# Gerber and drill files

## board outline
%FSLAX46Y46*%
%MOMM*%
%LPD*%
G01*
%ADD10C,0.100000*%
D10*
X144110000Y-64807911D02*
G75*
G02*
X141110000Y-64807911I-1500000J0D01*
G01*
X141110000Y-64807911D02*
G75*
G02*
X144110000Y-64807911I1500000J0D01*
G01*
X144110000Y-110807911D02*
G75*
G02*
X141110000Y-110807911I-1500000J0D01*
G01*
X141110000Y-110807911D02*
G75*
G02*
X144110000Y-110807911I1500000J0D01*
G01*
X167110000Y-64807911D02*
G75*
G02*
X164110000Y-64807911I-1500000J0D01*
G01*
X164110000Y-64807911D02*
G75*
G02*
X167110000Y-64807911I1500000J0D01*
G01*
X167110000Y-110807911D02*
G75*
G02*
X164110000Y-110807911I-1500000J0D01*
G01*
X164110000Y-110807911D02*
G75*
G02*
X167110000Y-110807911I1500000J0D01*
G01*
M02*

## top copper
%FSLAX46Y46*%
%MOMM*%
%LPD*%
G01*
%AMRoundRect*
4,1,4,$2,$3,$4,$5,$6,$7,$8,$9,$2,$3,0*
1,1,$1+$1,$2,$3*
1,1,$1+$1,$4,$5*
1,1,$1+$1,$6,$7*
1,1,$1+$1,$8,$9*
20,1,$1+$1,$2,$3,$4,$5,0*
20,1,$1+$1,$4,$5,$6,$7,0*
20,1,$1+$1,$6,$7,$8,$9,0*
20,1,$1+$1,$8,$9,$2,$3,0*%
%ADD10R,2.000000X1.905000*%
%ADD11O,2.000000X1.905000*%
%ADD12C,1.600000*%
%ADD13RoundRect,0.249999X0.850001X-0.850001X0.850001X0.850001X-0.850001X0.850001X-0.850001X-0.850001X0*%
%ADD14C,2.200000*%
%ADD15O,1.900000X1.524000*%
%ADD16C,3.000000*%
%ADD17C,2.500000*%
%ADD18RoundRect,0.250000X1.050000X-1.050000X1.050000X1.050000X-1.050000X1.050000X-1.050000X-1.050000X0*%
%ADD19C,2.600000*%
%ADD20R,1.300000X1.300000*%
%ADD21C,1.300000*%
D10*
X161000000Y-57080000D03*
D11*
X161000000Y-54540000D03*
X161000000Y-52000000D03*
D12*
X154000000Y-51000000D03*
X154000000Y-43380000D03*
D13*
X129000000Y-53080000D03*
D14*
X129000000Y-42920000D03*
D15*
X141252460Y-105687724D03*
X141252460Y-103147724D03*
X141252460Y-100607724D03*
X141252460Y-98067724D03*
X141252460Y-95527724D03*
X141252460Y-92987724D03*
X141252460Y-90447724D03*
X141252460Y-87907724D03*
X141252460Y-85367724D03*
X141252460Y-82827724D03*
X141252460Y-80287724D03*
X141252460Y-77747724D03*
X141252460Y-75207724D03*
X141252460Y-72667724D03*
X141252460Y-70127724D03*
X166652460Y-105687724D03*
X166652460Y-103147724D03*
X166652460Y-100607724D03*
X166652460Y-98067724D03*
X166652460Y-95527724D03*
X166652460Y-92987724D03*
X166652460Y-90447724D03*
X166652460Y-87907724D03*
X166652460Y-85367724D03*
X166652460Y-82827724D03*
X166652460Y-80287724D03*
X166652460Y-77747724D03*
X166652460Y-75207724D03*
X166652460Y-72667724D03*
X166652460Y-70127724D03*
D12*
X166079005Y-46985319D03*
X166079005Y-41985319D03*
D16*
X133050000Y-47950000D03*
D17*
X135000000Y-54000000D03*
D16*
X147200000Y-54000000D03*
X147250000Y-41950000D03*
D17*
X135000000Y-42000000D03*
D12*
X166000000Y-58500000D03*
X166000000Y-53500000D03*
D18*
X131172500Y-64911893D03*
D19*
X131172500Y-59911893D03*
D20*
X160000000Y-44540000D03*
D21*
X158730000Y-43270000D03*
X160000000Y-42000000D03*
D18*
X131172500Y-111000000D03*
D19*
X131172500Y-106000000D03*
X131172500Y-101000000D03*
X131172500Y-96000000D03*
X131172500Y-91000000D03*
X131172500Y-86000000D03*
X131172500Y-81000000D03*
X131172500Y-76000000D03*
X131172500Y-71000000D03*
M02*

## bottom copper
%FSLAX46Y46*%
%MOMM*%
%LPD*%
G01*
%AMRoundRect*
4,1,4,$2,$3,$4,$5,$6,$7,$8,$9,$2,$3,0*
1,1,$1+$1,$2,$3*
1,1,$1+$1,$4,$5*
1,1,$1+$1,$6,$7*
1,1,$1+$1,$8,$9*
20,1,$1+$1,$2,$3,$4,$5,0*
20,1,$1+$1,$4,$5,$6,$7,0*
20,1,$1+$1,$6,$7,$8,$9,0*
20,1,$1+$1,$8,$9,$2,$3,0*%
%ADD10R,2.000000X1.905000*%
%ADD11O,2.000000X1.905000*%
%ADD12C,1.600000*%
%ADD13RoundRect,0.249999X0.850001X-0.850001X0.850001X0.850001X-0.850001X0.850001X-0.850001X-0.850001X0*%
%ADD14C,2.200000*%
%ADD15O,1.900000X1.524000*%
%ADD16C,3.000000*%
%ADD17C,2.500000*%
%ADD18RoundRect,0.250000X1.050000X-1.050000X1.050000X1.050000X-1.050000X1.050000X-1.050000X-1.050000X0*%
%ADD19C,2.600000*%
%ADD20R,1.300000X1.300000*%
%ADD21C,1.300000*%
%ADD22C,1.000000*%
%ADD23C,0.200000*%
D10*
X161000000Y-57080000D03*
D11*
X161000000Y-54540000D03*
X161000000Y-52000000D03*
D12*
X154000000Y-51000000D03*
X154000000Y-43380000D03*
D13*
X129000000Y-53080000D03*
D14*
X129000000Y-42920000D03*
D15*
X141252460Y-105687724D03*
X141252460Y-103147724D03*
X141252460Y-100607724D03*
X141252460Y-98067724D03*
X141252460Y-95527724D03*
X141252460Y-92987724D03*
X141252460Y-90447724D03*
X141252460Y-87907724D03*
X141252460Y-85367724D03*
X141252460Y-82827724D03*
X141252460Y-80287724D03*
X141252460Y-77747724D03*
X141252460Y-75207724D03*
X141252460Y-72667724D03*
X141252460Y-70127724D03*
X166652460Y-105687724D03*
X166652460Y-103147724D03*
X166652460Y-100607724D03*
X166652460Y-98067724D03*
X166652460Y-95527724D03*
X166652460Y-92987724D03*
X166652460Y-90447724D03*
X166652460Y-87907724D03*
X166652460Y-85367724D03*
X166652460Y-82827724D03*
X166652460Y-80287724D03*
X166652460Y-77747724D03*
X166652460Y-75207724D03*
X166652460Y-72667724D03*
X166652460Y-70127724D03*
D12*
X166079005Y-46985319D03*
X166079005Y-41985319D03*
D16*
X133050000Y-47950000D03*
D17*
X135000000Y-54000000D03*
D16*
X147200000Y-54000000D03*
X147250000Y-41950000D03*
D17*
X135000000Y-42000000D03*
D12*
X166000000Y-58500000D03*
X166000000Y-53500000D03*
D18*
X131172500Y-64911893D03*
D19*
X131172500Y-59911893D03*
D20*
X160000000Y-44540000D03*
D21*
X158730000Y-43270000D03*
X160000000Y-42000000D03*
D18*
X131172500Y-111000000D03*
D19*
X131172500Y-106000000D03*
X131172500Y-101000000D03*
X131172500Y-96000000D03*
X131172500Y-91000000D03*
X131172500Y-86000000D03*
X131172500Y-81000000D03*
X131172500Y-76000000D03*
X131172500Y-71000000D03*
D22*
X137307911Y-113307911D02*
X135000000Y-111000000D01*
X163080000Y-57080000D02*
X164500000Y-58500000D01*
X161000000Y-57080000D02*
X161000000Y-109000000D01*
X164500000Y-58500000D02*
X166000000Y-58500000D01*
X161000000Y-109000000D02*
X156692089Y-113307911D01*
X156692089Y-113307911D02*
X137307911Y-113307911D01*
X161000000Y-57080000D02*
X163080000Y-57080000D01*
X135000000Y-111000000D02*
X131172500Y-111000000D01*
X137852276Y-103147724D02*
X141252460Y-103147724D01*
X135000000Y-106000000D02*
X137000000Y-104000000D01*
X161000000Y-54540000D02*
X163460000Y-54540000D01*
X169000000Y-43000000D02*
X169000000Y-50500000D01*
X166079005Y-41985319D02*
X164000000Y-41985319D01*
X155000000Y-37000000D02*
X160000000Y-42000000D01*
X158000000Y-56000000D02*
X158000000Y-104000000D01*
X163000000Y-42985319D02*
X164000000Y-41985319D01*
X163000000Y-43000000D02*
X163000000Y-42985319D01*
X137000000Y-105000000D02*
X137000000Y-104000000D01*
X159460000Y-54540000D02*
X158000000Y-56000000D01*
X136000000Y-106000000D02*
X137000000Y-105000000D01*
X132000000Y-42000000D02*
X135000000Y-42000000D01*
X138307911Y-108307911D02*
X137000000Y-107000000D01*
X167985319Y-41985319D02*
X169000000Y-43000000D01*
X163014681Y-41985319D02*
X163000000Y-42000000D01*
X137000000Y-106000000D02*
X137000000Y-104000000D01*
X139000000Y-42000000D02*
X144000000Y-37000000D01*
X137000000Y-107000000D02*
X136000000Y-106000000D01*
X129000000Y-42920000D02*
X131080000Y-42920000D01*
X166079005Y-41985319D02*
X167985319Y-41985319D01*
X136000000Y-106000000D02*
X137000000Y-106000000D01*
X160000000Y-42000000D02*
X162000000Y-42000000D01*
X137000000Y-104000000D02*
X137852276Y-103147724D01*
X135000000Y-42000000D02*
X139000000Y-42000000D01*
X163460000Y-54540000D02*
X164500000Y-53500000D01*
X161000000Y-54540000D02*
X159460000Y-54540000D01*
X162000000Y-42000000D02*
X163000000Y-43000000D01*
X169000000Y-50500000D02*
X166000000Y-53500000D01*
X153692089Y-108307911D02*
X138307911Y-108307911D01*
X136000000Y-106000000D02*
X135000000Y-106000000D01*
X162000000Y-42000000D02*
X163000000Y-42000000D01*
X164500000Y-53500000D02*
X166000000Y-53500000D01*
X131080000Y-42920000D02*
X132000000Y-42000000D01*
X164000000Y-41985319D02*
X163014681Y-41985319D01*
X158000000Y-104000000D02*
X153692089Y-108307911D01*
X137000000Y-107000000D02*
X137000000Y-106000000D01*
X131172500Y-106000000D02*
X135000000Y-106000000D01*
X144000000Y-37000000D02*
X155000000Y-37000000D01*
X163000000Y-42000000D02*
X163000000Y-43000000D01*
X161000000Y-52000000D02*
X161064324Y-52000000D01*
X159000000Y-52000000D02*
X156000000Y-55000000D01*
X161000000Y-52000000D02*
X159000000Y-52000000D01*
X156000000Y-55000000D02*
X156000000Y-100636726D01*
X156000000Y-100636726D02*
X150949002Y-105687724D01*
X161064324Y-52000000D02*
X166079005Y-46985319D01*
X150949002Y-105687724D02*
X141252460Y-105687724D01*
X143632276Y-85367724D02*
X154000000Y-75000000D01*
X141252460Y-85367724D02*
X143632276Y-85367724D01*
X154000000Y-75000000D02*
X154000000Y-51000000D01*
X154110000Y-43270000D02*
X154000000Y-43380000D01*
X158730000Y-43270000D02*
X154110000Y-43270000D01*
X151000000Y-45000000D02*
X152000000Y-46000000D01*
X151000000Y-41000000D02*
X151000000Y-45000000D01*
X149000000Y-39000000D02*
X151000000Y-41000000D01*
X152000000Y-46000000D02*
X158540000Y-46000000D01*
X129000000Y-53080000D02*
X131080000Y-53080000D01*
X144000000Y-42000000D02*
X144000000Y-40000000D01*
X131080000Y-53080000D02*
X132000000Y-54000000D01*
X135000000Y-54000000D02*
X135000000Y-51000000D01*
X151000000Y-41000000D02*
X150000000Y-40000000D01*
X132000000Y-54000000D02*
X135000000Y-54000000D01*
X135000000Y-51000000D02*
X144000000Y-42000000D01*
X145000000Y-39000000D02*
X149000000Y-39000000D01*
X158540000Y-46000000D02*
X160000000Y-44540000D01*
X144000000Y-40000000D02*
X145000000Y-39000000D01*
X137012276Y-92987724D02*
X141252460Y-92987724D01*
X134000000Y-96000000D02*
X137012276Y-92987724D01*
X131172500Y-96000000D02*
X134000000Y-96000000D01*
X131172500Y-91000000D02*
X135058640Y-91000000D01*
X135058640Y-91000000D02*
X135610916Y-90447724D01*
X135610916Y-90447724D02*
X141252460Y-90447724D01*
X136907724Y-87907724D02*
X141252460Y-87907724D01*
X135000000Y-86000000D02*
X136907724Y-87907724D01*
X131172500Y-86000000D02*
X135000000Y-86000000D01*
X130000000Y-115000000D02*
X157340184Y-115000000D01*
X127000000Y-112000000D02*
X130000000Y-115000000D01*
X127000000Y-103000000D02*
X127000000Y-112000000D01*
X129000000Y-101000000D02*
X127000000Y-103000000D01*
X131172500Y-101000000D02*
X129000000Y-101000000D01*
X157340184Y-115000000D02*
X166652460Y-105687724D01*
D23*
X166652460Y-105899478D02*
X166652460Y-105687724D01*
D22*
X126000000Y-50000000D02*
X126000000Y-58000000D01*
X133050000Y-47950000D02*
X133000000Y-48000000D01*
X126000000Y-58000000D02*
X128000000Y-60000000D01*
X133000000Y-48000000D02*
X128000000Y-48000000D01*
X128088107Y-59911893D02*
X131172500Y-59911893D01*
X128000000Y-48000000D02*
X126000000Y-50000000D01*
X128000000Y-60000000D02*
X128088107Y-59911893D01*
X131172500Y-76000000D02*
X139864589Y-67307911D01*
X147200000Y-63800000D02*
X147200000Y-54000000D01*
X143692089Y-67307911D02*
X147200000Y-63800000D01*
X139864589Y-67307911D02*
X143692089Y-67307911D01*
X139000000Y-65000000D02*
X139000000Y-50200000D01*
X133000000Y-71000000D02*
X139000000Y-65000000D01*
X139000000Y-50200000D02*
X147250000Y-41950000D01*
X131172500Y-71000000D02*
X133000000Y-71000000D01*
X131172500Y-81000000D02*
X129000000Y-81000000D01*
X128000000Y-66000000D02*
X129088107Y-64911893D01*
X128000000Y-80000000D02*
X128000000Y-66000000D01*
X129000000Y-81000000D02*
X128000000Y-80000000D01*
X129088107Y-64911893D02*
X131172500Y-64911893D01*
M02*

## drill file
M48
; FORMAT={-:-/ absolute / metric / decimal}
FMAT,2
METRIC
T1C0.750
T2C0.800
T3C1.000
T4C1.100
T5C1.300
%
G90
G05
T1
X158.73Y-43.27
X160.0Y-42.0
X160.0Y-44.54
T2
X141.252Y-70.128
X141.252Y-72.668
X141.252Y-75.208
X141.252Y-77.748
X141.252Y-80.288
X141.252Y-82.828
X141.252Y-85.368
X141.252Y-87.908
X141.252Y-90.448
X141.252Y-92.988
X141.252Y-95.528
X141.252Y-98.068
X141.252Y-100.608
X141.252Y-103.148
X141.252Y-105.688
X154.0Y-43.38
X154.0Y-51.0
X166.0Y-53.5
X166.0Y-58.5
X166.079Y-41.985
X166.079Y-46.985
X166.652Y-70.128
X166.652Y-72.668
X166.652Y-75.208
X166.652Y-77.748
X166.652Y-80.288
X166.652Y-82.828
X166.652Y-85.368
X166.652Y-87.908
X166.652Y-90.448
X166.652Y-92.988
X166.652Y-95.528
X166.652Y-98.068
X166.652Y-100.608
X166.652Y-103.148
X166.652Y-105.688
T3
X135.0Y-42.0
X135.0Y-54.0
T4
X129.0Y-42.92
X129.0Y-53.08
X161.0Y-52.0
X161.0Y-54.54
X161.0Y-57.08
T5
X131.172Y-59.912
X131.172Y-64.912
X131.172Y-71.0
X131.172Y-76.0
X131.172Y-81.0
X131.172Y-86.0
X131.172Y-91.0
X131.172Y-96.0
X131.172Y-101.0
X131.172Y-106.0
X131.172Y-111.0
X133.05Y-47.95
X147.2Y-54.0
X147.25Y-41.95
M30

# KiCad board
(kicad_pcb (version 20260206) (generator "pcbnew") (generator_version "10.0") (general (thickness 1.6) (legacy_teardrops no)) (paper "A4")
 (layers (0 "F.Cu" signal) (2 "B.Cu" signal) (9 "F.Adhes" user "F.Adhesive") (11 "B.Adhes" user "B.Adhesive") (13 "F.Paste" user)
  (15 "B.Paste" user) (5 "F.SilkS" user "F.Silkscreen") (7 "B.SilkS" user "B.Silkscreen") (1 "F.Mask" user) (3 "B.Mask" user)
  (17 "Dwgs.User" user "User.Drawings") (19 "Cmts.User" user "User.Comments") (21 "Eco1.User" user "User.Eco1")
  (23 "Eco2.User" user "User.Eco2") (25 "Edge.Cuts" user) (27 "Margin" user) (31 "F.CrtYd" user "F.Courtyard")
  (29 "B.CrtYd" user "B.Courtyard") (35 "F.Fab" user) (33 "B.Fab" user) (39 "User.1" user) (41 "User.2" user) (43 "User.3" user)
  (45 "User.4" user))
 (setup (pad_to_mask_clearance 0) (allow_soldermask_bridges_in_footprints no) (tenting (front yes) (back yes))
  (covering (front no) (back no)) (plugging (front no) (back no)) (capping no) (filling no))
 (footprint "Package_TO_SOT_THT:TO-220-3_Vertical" (layer "F.Cu") (at 161 57.08 90)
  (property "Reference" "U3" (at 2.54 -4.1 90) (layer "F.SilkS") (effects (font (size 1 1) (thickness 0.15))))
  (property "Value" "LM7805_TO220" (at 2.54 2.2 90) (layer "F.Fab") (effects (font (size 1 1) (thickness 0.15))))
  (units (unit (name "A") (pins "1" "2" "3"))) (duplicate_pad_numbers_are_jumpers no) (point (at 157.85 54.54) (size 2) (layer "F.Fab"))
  (pad "1" thru_hole rect (at 0 0 90) (size 1.905 2) (drill 1.1) (layers "*.Cu" "*.Mask") (remove_unused_layers no) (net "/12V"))
  (pad "2" thru_hole oval (at 2.54 0 90) (size 1.905 2) (drill 1.1) (layers "*.Cu" "*.Mask") (remove_unused_layers no) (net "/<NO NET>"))
  (pad "3" thru_hole oval (at 5.08 0 90) (size 1.905 2) (drill 1.1) (layers "*.Cu" "*.Mask") (remove_unused_layers no) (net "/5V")))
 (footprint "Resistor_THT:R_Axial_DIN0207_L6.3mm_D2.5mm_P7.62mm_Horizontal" (layer "F.Cu") (at 154 51 90)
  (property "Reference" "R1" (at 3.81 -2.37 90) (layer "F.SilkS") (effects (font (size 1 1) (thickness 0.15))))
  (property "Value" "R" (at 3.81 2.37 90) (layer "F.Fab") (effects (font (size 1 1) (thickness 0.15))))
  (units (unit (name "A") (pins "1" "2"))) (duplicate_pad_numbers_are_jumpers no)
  (pad "1" thru_hole circle (at 0 0 90) (size 1.6 1.6) (drill 0.8) (layers "*.Cu" "*.Mask") (remove_unused_layers no)
   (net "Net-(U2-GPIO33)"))
  (pad "2" thru_hole circle (at 7.62 0 90) (size 1.6 1.6) (drill 0.8) (layers "*.Cu" "*.Mask") (remove_unused_layers no) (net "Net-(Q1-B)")))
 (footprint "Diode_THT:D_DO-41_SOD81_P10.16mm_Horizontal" (layer "F.Cu") (at 129 53.08 90)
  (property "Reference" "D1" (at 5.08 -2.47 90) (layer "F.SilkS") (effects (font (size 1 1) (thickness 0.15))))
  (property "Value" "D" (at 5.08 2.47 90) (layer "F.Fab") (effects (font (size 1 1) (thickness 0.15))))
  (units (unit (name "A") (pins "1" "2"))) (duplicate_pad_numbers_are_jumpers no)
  (pad "1" thru_hole roundrect (at 0 0 90) (size 2.2 2.2) (drill 1.1) (layers "*.Cu" "*.Mask") (remove_unused_layers no)
   (roundrect_rratio 0.113636) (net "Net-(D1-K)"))
  (pad "2" thru_hole circle (at 10.16 0 90) (size 2.2 2.2) (drill 1.1) (layers "*.Cu" "*.Mask") (remove_unused_layers no) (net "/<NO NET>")))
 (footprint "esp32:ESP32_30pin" (layer "F.Cu") (at 153.18 88.667911)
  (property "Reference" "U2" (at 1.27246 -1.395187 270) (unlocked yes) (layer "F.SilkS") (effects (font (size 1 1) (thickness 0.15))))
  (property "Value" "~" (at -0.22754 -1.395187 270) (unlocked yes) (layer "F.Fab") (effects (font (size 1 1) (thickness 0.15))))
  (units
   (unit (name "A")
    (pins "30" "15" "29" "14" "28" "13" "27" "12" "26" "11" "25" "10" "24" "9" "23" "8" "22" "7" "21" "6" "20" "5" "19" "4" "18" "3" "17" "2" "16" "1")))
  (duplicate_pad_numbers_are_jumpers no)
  (fp_circle (center -10.57 -23.86) (end -10.57 -22.36) (stroke (width 0.1) (type default)) (fill no) (layer "Edge.Cuts"))
  (fp_circle (center -10.57 22.14) (end -10.57 23.64) (stroke (width 0.1) (type default)) (fill no) (layer "Edge.Cuts"))
  (fp_circle (center 12.43 -23.86) (end 12.43 -22.36) (stroke (width 0.1) (type default)) (fill no) (layer "Edge.Cuts"))
  (fp_circle (center 12.43 22.14) (end 12.43 23.64) (stroke (width 0.1) (type default)) (fill no) (layer "Edge.Cuts"))
  (pad "1" thru_hole oval (at -11.92754 17.019813 270) (size 1.524 1.9) (drill 0.8) (layers "*.Cu" "*.Mask") (remove_unused_layers no)
   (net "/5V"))
  (pad "2" thru_hole oval (at -11.92754 14.479813 270) (size 1.524 1.9) (drill 0.8) (layers "*.Cu" "*.Mask") (remove_unused_layers no)
   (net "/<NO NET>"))
  (pad "3" thru_hole oval (at -11.92754 11.939813 270) (size 1.524 1.9) (drill 0.8) (layers "*.Cu" "*.Mask") (remove_unused_layers no)
   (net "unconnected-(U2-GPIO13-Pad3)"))
  (pad "4" thru_hole oval (at -11.92754 9.399813 270) (size 1.524 1.9) (drill 0.8) (layers "*.Cu" "*.Mask") (remove_unused_layers no)
   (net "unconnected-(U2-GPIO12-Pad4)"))
  (pad "5" thru_hole oval (at -11.92754 6.859813 270) (size 1.524 1.9) (drill 0.8) (layers "*.Cu" "*.Mask") (remove_unused_layers no)
   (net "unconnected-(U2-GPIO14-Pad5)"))
  (pad "6" thru_hole oval (at -11.92754 4.319813 270) (size 1.524 1.9) (drill 0.8) (layers "*.Cu" "*.Mask") (remove_unused_layers no)
   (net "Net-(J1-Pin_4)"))
  (pad "7" thru_hole oval (at -11.92754 1.779813 270) (size 1.524 1.9) (drill 0.8) (layers "*.Cu" "*.Mask") (remove_unused_layers no)
   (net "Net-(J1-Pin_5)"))
  (pad "8" thru_hole oval (at -11.92754 -0.760187 270) (size 1.524 1.9) (drill 0.8) (layers "*.Cu" "*.Mask") (remove_unused_layers no)
   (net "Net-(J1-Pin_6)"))
  (pad "9" thru_hole oval (at -11.92754 -3.300187 270) (size 1.524 1.9) (drill 0.8) (layers "*.Cu" "*.Mask") (remove_unused_layers no)
   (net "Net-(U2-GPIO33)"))
  (pad "10" thru_hole oval (at -11.92754 -5.840187 270) (size 1.524 1.9) (drill 0.8) (layers "*.Cu" "*.Mask") (remove_unused_layers no)
   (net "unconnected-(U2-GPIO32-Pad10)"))
  (pad "11" thru_hole oval (at -11.92754 -8.380187 270) (size 1.524 1.9) (drill 0.8) (layers "*.Cu" "*.Mask") (remove_unused_layers no)
   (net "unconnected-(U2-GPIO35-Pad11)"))
  (pad "12" thru_hole oval (at -11.92754 -10.920187 270) (size 1.524 1.9) (drill 0.8) (layers "*.Cu" "*.Mask") (remove_unused_layers no)
   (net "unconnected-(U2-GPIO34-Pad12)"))
  (pad "13" thru_hole oval (at -11.92754 -13.460187 270) (size 1.524 1.9) (drill 0.8) (layers "*.Cu" "*.Mask") (remove_unused_layers no)
   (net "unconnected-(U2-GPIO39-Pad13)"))
  (pad "14" thru_hole oval (at -11.92754 -16.000187 270) (size 1.524 1.9) (drill 0.8) (layers "*.Cu" "*.Mask") (remove_unused_layers no)
   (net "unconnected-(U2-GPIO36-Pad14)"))
  (pad "15" thru_hole oval (at -11.92754 -18.540187 270) (size 1.524 1.9) (drill 0.8) (layers "*.Cu" "*.Mask") (remove_unused_layers no)
   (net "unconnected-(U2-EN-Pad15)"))
  (pad "16" thru_hole oval (at 13.47246 17.019813 270) (size 1.524 1.9) (drill 0.8) (layers "*.Cu" "*.Mask") (remove_unused_layers no)
   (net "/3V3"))
  (pad "17" thru_hole oval (at 13.47246 14.479813 270) (size 1.524 1.9) (drill 0.8) (layers "*.Cu" "*.Mask") (remove_unused_layers no)
   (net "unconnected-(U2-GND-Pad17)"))
  (pad "18" thru_hole oval (at 13.47246 11.939813 270) (size 1.524 1.9) (drill 0.8) (layers "*.Cu" "*.Mask") (remove_unused_layers no)
   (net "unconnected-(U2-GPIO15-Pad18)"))
  (pad "19" thru_hole oval (at 13.47246 9.399813 270) (size 1.524 1.9) (drill 0.8) (layers "*.Cu" "*.Mask") (remove_unused_layers no)
   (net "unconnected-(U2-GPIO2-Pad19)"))
  (pad "20" thru_hole oval (at 13.47246 6.859813 270) (size 1.524 1.9) (drill 0.8) (layers "*.Cu" "*.Mask" "Dwgs.User")
   (remove_unused_layers no) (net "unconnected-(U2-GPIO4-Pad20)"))
  (pad "21" thru_hole oval (at 13.47246 4.319813 270) (size 1.524 1.9) (drill 0.8) (layers "*.Cu" "*.Mask") (remove_unused_layers no)
   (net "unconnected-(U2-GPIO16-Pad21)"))
  (pad "22" thru_hole oval (at 13.47246 1.779813 270) (size 1.524 1.9) (drill 0.8) (layers "*.Cu" "*.Mask") (remove_unused_layers no)
   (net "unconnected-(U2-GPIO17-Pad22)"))
  (pad "23" thru_hole oval (at 13.47246 -0.760187 270) (size 1.524 1.9) (drill 0.8) (layers "*.Cu" "*.Mask") (remove_unused_layers no)
   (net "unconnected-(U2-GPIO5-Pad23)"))
  (pad "24" thru_hole oval (at 13.47246 -3.300187 270) (size 1.524 1.9) (drill 0.8) (layers "*.Cu" "*.Mask") (remove_unused_layers no)
   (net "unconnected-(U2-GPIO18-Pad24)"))
  (pad "25" thru_hole oval (at 13.47246 -5.840187 270) (size 1.524 1.9) (drill 0.8) (layers "*.Cu" "*.Mask") (remove_unused_layers no)
   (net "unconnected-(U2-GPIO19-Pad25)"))
  (pad "26" thru_hole oval (at 13.47246 -8.380187 270) (size 1.524 1.9) (drill 0.8) (layers "*.Cu" "*.Mask") (remove_unused_layers no)
   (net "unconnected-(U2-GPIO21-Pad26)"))
  (pad "27" thru_hole oval (at 13.47246 -10.920187 270) (size 1.524 1.9) (drill 0.8) (layers "*.Cu" "*.Mask") (remove_unused_layers no)
   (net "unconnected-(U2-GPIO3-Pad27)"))
  (pad "28" thru_hole oval (at 13.47246 -13.460187 270) (size 1.524 1.9) (drill 0.8) (layers "*.Cu" "*.Mask") (remove_unused_layers no)
   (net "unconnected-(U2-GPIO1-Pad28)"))
  (pad "29" thru_hole oval (at 13.47246 -16.000187 270) (size 1.524 1.9) (drill 0.8) (layers "*.Cu" "*.Mask") (remove_unused_layers no)
   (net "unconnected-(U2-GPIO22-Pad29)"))
  (pad "30" thru_hole oval (at 13.47246 -18.540187 270) (size 1.524 1.9) (drill 0.8) (layers "*.Cu" "*.Mask") (remove_unused_layers no)
   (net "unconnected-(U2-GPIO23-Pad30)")))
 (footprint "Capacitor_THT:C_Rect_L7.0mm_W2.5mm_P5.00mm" (layer "F.Cu") (at 166.079005 46.985319 90)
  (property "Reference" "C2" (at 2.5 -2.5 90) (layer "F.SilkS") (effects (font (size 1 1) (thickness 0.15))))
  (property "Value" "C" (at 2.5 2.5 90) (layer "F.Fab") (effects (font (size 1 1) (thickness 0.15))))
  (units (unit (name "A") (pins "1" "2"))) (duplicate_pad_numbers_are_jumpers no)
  (pad "1" thru_hole circle (at 0 0 90) (size 1.6 1.6) (drill 0.8) (layers "*.Cu" "*.Mask") (remove_unused_layers no) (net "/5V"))
  (pad "2" thru_hole circle (at 5 0 90) (size 1.6 1.6) (drill 0.8) (layers "*.Cu" "*.Mask") (remove_unused_layers no) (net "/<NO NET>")))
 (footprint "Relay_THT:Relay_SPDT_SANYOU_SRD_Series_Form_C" (layer "F.Cu") (at 133.05 47.95)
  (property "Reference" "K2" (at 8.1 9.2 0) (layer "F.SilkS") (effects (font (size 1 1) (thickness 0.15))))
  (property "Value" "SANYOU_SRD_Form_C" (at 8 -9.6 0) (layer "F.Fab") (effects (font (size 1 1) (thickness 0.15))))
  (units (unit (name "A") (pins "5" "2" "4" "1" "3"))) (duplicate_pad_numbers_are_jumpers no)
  (pad "1" thru_hole circle (at 0 0 90) (size 3 3) (drill 1.3) (layers "*.Cu" "*.Mask") (remove_unused_layers no) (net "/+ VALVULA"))
  (pad "2" thru_hole circle (at 1.95 6.05 90) (size 2.5 2.5) (drill 1) (layers "*.Cu" "*.Mask") (remove_unused_layers no) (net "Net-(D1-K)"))
  (pad "3" thru_hole circle (at 14.15 6.05 90) (size 3 3) (drill 1.3) (layers "*.Cu" "*.Mask") (remove_unused_layers no) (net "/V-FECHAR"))
  (pad "4" thru_hole circle (at 14.2 -6 90) (size 3 3) (drill 1.3) (layers "*.Cu" "*.Mask") (remove_unused_layers no) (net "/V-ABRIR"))
  (pad "5" thru_hole circle (at 1.95 -5.95 90) (size 2.5 2.5) (drill 1) (layers "*.Cu" "*.Mask") (remove_unused_layers no) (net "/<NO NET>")))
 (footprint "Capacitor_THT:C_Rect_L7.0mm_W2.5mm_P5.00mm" (layer "F.Cu") (at 166 58.5 90)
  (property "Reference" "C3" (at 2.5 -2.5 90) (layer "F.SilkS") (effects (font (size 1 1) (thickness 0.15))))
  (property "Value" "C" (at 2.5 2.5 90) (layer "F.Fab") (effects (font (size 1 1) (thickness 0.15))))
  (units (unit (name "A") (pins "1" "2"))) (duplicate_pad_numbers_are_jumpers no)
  (pad "1" thru_hole circle (at 0 0 90) (size 1.6 1.6) (drill 0.8) (layers "*.Cu" "*.Mask") (remove_unused_layers no) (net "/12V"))
  (pad "2" thru_hole circle (at 5 0 90) (size 1.6 1.6) (drill 0.8) (layers "*.Cu" "*.Mask") (remove_unused_layers no) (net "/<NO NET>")))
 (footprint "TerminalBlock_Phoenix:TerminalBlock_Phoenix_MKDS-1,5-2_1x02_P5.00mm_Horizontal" (layer "F.Cu") (at 131.1725 64.911893 90)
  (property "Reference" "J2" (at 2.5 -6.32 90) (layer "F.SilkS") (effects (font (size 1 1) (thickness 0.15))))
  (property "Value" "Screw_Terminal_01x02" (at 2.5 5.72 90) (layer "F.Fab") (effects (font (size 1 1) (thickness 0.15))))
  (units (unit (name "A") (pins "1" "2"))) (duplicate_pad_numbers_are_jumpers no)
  (pad "1" thru_hole roundrect (at 0 0 90) (size 2.6 2.6) (drill 1.3) (layers "*.Cu" "*.Mask") (remove_unused_layers no)
   (roundrect_rratio 0.096154) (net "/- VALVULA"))
  (pad "2" thru_hole circle (at 5 0 90) (size 2.6 2.6) (drill 1.3) (layers "*.Cu" "*.Mask") (remove_unused_layers no) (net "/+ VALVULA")))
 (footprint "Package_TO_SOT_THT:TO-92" (layer "F.Cu") (at 160 44.54 90)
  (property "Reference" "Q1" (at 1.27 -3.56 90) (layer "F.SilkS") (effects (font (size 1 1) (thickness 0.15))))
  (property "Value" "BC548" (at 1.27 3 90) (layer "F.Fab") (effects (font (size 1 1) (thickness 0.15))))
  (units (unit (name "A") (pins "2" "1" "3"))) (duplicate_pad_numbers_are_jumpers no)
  (pad "1" thru_hole rect (at 0 0 90) (size 1.3 1.3) (drill 0.75) (layers "*.Cu" "*.Mask") (remove_unused_layers no) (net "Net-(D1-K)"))
  (pad "2" thru_hole circle (at 1.27 -1.27 90) (size 1.3 1.3) (drill 0.75) (layers "*.Cu" "*.Mask") (remove_unused_layers no)
   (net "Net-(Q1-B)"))
  (pad "3" thru_hole circle (at 2.54 0 90) (size 1.3 1.3) (drill 0.75) (layers "*.Cu" "*.Mask") (remove_unused_layers no) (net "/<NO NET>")))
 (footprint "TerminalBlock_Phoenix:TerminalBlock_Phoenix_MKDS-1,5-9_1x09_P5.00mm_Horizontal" (layer "F.Cu") (at 131.1725 111 90)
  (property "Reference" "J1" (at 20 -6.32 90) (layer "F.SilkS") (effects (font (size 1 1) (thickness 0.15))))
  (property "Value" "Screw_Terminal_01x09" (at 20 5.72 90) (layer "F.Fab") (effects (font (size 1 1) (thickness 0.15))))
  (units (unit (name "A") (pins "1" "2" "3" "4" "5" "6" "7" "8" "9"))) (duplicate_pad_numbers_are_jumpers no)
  (pad "1" thru_hole roundrect (at 0 0 90) (size 2.6 2.6) (drill 1.3) (layers "*.Cu" "*.Mask") (remove_unused_layers no)
   (roundrect_rratio 0.096154) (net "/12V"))
  (pad "2" thru_hole circle (at 5 0 90) (size 2.6 2.6) (drill 1.3) (layers "*.Cu" "*.Mask") (remove_unused_layers no) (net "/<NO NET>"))
  (pad "3" thru_hole circle (at 10 0 90) (size 2.6 2.6) (drill 1.3) (layers "*.Cu" "*.Mask") (remove_unused_layers no) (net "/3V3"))
  (pad "4" thru_hole circle (at 15 0 90) (size 2.6 2.6) (drill 1.3) (layers "*.Cu" "*.Mask") (remove_unused_layers no)
   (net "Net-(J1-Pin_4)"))
  (pad "5" thru_hole circle (at 20 0 90) (size 2.6 2.6) (drill 1.3) (layers "*.Cu" "*.Mask") (remove_unused_layers no)
   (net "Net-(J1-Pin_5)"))
  (pad "6" thru_hole circle (at 25 0 90) (size 2.6 2.6) (drill 1.3) (layers "*.Cu" "*.Mask") (remove_unused_layers no)
   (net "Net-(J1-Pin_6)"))
  (pad "7" thru_hole circle (at 30 0 90) (size 2.6 2.6) (drill 1.3) (layers "*.Cu" "*.Mask") (remove_unused_layers no) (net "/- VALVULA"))
  (pad "8" thru_hole circle (at 35 0 90) (size 2.6 2.6) (drill 1.3) (layers "*.Cu" "*.Mask") (remove_unused_layers no) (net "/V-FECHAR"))
  (pad "9" thru_hole circle (at 40 0 90) (size 2.6 2.6) (drill 1.3) (layers "*.Cu" "*.Mask") (remove_unused_layers no) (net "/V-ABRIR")))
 (segment (start 137.307911 113.307911) (end 135 111) (width 1) (layer "B.Cu") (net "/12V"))
 (segment (start 163.08 57.08) (end 164.5 58.5) (width 1) (layer "B.Cu") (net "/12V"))
 (segment (start 161 57.08) (end 161 109) (width 1) (layer "B.Cu") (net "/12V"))
 (segment (start 164.5 58.5) (end 166 58.5) (width 1) (layer "B.Cu") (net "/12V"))
 (segment (start 161 109) (end 156.692089 113.307911) (width 1) (layer "B.Cu") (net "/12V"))
 (segment (start 156.692089 113.307911) (end 137.307911 113.307911) (width 1) (layer "B.Cu") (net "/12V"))
 (segment (start 161 57.08) (end 163.08 57.08) (width 1) (layer "B.Cu") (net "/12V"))
 (segment (start 135 111) (end 131.1725 111) (width 1) (layer "B.Cu") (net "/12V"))
 (segment (start 137.852276 103.147724) (end 141.25246 103.147724) (width 1) (layer "B.Cu") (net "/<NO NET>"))
 (segment (start 135 106) (end 137 104) (width 1) (layer "B.Cu") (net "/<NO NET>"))
 (segment (start 161 54.54) (end 163.46 54.54) (width 1) (layer "B.Cu") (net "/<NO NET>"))
 (segment (start 169 43) (end 169 50.5) (width 1) (layer "B.Cu") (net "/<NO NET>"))
 (segment (start 166.079005 41.985319) (end 164 41.985319) (width 1) (layer "B.Cu") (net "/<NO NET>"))
 (segment (start 155 37) (end 160 42) (width 1) (layer "B.Cu") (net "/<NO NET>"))
 (segment (start 158 56) (end 158 104) (width 1) (layer "B.Cu") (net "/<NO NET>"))
 (segment (start 163 42.985319) (end 164 41.985319) (width 1) (layer "B.Cu") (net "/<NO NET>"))
 (segment (start 163 43) (end 163 42.985319) (width 1) (layer "B.Cu") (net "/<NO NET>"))
 (segment (start 137 105) (end 137 104) (width 1) (layer "B.Cu") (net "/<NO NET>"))
 (segment (start 159.46 54.54) (end 158 56) (width 1) (layer "B.Cu") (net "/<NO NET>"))
 (segment (start 136 106) (end 137 105) (width 1) (layer "B.Cu") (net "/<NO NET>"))
 (segment (start 132 42) (end 135 42) (width 1) (layer "B.Cu") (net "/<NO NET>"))
 (segment (start 138.307911 108.307911) (end 137 107) (width 1) (layer "B.Cu") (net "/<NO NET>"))
 (segment (start 167.985319 41.985319) (end 169 43) (width 1) (layer "B.Cu") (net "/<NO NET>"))
 (segment (start 163.014681 41.985319) (end 163 42) (width 1) (layer "B.Cu") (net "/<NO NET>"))
 (segment (start 137 106) (end 137 104) (width 1) (layer "B.Cu") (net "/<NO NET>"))
 (segment (start 139 42) (end 144 37) (width 1) (layer "B.Cu") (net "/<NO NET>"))
 (segment (start 137 107) (end 136 106) (width 1) (layer "B.Cu") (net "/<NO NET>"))
 (segment (start 129 42.92) (end 131.08 42.92) (width 1) (layer "B.Cu") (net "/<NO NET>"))
 (segment (start 166.079005 41.985319) (end 167.985319 41.985319) (width 1) (layer "B.Cu") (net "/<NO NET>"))
 (segment (start 136 106) (end 137 106) (width 1) (layer "B.Cu") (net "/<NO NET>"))
 (segment (start 160 42) (end 162 42) (width 1) (layer "B.Cu") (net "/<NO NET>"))
 (segment (start 137 104) (end 137.852276 103.147724) (width 1) (layer "B.Cu") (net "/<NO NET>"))
 (segment (start 135 42) (end 139 42) (width 1) (layer "B.Cu") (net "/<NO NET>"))
 (segment (start 163.46 54.54) (end 164.5 53.5) (width 1) (layer "B.Cu") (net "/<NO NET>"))
 (segment (start 161 54.54) (end 159.46 54.54) (width 1) (layer "B.Cu") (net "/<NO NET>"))
 (segment (start 162 42) (end 163 43) (width 1) (layer "B.Cu") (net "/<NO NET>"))
 (segment (start 169 50.5) (end 166 53.5) (width 1) (layer "B.Cu") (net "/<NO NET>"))
 (segment (start 153.692089 108.307911) (end 138.307911 108.307911) (width 1) (layer "B.Cu") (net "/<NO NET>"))
 (segment (start 136 106) (end 135 106) (width 1) (layer "B.Cu") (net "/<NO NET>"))
 (segment (start 162 42) (end 163 42) (width 1) (layer "B.Cu") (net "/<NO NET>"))
 (segment (start 164.5 53.5) (end 166 53.5) (width 1) (layer "B.Cu") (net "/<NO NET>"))
 (segment (start 131.08 42.92) (end 132 42) (width 1) (layer "B.Cu") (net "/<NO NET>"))
 (segment (start 164 41.985319) (end 163.014681 41.985319) (width 1) (layer "B.Cu") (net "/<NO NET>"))
 (segment (start 158 104) (end 153.692089 108.307911) (width 1) (layer "B.Cu") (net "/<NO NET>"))
 (segment (start 137 107) (end 137 106) (width 1) (layer "B.Cu") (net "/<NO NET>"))
 (segment (start 131.1725 106) (end 135 106) (width 1) (layer "B.Cu") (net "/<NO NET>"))
 (segment (start 144 37) (end 155 37) (width 1) (layer "B.Cu") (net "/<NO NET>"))
 (segment (start 163 42) (end 163 43) (width 1) (layer "B.Cu") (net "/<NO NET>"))
 (segment (start 161 52) (end 161.064324 52) (width 1) (layer "B.Cu") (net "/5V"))
 (segment (start 159 52) (end 156 55) (width 1) (layer "B.Cu") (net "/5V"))
 (segment (start 161 52) (end 159 52) (width 1) (layer "B.Cu") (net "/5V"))
 (segment (start 156 55) (end 156 100.636726) (width 1) (layer "B.Cu") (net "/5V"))
 (segment (start 156 100.636726) (end 150.949002 105.687724) (width 1) (layer "B.Cu") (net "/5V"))
 (segment (start 161.064324 52) (end 166.079005 46.985319) (width 1) (layer "B.Cu") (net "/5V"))
 (segment (start 150.949002 105.687724) (end 141.25246 105.687724) (width 1) (layer "B.Cu") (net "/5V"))
 (segment (start 143.632276 85.367724) (end 154 75) (width 1) (layer "B.Cu") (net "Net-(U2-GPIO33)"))
 (segment (start 141.25246 85.367724) (end 143.632276 85.367724) (width 1) (layer "B.Cu") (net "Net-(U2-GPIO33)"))
 (segment (start 154 75) (end 154 51) (width 1) (layer "B.Cu") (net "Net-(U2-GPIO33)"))
 (segment (start 154.11 43.27) (end 154 43.38) (width 1) (layer "B.Cu") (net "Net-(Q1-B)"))
 (segment (start 158.73 43.27) (end 154.11 43.27) (width 1) (layer "B.Cu") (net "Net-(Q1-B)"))
 (segment (start 151 45) (end 152 46) (width 1) (layer "B.Cu") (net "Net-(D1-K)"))
 (segment (start 151 41) (end 151 45) (width 1) (layer "B.Cu") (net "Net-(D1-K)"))
 (segment (start 149 39) (end 151 41) (width 1) (layer "B.Cu") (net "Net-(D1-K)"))
 (segment (start 152 46) (end 158.54 46) (width 1) (layer "B.Cu") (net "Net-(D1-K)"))
 (segment (start 129 53.08) (end 131.08 53.08) (width 1) (layer "B.Cu") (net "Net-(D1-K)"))
 (segment (start 144 42) (end 144 40) (width 1) (layer "B.Cu") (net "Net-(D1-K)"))
 (segment (start 131.08 53.08) (end 132 54) (width 1) (layer "B.Cu") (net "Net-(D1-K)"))
 (segment (start 135 54) (end 135 51) (width 1) (layer "B.Cu") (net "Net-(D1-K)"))
 (segment (start 151 41) (end 150 40) (width 1) (layer "B.Cu") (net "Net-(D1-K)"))
 (segment (start 132 54) (end 135 54) (width 1) (layer "B.Cu") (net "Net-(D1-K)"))
 (segment (start 135 51) (end 144 42) (width 1) (layer "B.Cu") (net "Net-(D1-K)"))
 (segment (start 145 39) (end 149 39) (width 1) (layer "B.Cu") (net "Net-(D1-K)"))
 (segment (start 158.54 46) (end 160 44.54) (width 1) (layer "B.Cu") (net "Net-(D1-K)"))
 (segment (start 144 40) (end 145 39) (width 1) (layer "B.Cu") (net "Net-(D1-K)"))
 (segment (start 137.012276 92.987724) (end 141.25246 92.987724) (width 1) (layer "B.Cu") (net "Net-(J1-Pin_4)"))
 (segment (start 134 96) (end 137.012276 92.987724) (width 1) (layer "B.Cu") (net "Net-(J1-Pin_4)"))
 (segment (start 131.1725 96) (end 134 96) (width 1) (layer "B.Cu") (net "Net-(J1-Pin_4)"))
 (segment (start 131.1725 91) (end 135.05864 91) (width 1) (layer "B.Cu") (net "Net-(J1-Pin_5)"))
 (segment (start 135.05864 91) (end 135.610916 90.447724) (width 1) (layer "B.Cu") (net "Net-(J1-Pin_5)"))
 (segment (start 135.610916 90.447724) (end 141.25246 90.447724) (width 1) (layer "B.Cu") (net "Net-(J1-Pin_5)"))
 (segment (start 136.907724 87.907724) (end 141.25246 87.907724) (width 1) (layer "B.Cu") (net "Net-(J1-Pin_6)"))
 (segment (start 135 86) (end 136.907724 87.907724) (width 1) (layer "B.Cu") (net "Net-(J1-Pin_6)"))
 (segment (start 131.1725 86) (end 135 86) (width 1) (layer "B.Cu") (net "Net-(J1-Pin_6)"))
 (segment (start 130 115) (end 157.340184 115) (width 1) (layer "B.Cu") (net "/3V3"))
 (segment (start 127 112) (end 130 115) (width 1) (layer "B.Cu") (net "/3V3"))
 (segment (start 127 103) (end 127 112) (width 1) (layer "B.Cu") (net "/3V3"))
 (segment (start 129 101) (end 127 103) (width 1) (layer "B.Cu") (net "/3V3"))
 (segment (start 131.1725 101) (end 129 101) (width 1) (layer "B.Cu") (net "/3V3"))
 (segment (start 157.340184 115) (end 166.65246 105.687724) (width 1) (layer "B.Cu") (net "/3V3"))
 (segment (start 166.65246 105.899478) (end 166.65246 105.687724) (width 0.2) (layer "B.Cu") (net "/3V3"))
 (segment (start 126 50) (end 126 58) (width 1) (layer "B.Cu") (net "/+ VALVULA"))
 (segment (start 133.05 47.95) (end 133 48) (width 1) (layer "B.Cu") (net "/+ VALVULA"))
 (segment (start 126 58) (end 128 60) (width 1) (layer "B.Cu") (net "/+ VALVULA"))
 (segment (start 133 48) (end 128 48) (width 1) (layer "B.Cu") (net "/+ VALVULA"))
 (segment (start 128.088107 59.911893) (end 131.1725 59.911893) (width 1) (layer "B.Cu") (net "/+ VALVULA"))
 (segment (start 128 48) (end 126 50) (width 1) (layer "B.Cu") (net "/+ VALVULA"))
 (segment (start 128 60) (end 128.088107 59.911893) (width 1) (layer "B.Cu") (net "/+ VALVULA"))
 (segment (start 131.1725 76) (end 139.864589 67.307911) (width 1) (layer "B.Cu") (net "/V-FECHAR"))
 (segment (start 147.2 63.8) (end 147.2 54) (width 1) (layer "B.Cu") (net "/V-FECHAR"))
 (segment (start 143.692089 67.307911) (end 147.2 63.8) (width 1) (layer "B.Cu") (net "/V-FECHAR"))
 (segment (start 139.864589 67.307911) (end 143.692089 67.307911) (width 1) (layer "B.Cu") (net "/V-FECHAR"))
 (segment (start 139 65) (end 139 50.2) (width 1) (layer "B.Cu") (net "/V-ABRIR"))
 (segment (start 133 71) (end 139 65) (width 1) (layer "B.Cu") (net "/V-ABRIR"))
 (segment (start 139 50.2) (end 147.25 41.95) (width 1) (layer "B.Cu") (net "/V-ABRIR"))
 (segment (start 131.1725 71) (end 133 71) (width 1) (layer "B.Cu") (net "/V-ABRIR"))
 (segment (start 131.1725 81) (end 129 81) (width 1) (layer "B.Cu") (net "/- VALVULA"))
 (segment (start 128 66) (end 129.088107 64.911893) (width 1) (layer "B.Cu") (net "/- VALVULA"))
 (segment (start 128 80) (end 128 66) (width 1) (layer "B.Cu") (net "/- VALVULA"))
 (segment (start 129 81) (end 128 80) (width 1) (layer "B.Cu") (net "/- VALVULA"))
 (segment (start 129.088107 64.911893) (end 131.1725 64.911893) (width 1) (layer "B.Cu") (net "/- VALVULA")))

